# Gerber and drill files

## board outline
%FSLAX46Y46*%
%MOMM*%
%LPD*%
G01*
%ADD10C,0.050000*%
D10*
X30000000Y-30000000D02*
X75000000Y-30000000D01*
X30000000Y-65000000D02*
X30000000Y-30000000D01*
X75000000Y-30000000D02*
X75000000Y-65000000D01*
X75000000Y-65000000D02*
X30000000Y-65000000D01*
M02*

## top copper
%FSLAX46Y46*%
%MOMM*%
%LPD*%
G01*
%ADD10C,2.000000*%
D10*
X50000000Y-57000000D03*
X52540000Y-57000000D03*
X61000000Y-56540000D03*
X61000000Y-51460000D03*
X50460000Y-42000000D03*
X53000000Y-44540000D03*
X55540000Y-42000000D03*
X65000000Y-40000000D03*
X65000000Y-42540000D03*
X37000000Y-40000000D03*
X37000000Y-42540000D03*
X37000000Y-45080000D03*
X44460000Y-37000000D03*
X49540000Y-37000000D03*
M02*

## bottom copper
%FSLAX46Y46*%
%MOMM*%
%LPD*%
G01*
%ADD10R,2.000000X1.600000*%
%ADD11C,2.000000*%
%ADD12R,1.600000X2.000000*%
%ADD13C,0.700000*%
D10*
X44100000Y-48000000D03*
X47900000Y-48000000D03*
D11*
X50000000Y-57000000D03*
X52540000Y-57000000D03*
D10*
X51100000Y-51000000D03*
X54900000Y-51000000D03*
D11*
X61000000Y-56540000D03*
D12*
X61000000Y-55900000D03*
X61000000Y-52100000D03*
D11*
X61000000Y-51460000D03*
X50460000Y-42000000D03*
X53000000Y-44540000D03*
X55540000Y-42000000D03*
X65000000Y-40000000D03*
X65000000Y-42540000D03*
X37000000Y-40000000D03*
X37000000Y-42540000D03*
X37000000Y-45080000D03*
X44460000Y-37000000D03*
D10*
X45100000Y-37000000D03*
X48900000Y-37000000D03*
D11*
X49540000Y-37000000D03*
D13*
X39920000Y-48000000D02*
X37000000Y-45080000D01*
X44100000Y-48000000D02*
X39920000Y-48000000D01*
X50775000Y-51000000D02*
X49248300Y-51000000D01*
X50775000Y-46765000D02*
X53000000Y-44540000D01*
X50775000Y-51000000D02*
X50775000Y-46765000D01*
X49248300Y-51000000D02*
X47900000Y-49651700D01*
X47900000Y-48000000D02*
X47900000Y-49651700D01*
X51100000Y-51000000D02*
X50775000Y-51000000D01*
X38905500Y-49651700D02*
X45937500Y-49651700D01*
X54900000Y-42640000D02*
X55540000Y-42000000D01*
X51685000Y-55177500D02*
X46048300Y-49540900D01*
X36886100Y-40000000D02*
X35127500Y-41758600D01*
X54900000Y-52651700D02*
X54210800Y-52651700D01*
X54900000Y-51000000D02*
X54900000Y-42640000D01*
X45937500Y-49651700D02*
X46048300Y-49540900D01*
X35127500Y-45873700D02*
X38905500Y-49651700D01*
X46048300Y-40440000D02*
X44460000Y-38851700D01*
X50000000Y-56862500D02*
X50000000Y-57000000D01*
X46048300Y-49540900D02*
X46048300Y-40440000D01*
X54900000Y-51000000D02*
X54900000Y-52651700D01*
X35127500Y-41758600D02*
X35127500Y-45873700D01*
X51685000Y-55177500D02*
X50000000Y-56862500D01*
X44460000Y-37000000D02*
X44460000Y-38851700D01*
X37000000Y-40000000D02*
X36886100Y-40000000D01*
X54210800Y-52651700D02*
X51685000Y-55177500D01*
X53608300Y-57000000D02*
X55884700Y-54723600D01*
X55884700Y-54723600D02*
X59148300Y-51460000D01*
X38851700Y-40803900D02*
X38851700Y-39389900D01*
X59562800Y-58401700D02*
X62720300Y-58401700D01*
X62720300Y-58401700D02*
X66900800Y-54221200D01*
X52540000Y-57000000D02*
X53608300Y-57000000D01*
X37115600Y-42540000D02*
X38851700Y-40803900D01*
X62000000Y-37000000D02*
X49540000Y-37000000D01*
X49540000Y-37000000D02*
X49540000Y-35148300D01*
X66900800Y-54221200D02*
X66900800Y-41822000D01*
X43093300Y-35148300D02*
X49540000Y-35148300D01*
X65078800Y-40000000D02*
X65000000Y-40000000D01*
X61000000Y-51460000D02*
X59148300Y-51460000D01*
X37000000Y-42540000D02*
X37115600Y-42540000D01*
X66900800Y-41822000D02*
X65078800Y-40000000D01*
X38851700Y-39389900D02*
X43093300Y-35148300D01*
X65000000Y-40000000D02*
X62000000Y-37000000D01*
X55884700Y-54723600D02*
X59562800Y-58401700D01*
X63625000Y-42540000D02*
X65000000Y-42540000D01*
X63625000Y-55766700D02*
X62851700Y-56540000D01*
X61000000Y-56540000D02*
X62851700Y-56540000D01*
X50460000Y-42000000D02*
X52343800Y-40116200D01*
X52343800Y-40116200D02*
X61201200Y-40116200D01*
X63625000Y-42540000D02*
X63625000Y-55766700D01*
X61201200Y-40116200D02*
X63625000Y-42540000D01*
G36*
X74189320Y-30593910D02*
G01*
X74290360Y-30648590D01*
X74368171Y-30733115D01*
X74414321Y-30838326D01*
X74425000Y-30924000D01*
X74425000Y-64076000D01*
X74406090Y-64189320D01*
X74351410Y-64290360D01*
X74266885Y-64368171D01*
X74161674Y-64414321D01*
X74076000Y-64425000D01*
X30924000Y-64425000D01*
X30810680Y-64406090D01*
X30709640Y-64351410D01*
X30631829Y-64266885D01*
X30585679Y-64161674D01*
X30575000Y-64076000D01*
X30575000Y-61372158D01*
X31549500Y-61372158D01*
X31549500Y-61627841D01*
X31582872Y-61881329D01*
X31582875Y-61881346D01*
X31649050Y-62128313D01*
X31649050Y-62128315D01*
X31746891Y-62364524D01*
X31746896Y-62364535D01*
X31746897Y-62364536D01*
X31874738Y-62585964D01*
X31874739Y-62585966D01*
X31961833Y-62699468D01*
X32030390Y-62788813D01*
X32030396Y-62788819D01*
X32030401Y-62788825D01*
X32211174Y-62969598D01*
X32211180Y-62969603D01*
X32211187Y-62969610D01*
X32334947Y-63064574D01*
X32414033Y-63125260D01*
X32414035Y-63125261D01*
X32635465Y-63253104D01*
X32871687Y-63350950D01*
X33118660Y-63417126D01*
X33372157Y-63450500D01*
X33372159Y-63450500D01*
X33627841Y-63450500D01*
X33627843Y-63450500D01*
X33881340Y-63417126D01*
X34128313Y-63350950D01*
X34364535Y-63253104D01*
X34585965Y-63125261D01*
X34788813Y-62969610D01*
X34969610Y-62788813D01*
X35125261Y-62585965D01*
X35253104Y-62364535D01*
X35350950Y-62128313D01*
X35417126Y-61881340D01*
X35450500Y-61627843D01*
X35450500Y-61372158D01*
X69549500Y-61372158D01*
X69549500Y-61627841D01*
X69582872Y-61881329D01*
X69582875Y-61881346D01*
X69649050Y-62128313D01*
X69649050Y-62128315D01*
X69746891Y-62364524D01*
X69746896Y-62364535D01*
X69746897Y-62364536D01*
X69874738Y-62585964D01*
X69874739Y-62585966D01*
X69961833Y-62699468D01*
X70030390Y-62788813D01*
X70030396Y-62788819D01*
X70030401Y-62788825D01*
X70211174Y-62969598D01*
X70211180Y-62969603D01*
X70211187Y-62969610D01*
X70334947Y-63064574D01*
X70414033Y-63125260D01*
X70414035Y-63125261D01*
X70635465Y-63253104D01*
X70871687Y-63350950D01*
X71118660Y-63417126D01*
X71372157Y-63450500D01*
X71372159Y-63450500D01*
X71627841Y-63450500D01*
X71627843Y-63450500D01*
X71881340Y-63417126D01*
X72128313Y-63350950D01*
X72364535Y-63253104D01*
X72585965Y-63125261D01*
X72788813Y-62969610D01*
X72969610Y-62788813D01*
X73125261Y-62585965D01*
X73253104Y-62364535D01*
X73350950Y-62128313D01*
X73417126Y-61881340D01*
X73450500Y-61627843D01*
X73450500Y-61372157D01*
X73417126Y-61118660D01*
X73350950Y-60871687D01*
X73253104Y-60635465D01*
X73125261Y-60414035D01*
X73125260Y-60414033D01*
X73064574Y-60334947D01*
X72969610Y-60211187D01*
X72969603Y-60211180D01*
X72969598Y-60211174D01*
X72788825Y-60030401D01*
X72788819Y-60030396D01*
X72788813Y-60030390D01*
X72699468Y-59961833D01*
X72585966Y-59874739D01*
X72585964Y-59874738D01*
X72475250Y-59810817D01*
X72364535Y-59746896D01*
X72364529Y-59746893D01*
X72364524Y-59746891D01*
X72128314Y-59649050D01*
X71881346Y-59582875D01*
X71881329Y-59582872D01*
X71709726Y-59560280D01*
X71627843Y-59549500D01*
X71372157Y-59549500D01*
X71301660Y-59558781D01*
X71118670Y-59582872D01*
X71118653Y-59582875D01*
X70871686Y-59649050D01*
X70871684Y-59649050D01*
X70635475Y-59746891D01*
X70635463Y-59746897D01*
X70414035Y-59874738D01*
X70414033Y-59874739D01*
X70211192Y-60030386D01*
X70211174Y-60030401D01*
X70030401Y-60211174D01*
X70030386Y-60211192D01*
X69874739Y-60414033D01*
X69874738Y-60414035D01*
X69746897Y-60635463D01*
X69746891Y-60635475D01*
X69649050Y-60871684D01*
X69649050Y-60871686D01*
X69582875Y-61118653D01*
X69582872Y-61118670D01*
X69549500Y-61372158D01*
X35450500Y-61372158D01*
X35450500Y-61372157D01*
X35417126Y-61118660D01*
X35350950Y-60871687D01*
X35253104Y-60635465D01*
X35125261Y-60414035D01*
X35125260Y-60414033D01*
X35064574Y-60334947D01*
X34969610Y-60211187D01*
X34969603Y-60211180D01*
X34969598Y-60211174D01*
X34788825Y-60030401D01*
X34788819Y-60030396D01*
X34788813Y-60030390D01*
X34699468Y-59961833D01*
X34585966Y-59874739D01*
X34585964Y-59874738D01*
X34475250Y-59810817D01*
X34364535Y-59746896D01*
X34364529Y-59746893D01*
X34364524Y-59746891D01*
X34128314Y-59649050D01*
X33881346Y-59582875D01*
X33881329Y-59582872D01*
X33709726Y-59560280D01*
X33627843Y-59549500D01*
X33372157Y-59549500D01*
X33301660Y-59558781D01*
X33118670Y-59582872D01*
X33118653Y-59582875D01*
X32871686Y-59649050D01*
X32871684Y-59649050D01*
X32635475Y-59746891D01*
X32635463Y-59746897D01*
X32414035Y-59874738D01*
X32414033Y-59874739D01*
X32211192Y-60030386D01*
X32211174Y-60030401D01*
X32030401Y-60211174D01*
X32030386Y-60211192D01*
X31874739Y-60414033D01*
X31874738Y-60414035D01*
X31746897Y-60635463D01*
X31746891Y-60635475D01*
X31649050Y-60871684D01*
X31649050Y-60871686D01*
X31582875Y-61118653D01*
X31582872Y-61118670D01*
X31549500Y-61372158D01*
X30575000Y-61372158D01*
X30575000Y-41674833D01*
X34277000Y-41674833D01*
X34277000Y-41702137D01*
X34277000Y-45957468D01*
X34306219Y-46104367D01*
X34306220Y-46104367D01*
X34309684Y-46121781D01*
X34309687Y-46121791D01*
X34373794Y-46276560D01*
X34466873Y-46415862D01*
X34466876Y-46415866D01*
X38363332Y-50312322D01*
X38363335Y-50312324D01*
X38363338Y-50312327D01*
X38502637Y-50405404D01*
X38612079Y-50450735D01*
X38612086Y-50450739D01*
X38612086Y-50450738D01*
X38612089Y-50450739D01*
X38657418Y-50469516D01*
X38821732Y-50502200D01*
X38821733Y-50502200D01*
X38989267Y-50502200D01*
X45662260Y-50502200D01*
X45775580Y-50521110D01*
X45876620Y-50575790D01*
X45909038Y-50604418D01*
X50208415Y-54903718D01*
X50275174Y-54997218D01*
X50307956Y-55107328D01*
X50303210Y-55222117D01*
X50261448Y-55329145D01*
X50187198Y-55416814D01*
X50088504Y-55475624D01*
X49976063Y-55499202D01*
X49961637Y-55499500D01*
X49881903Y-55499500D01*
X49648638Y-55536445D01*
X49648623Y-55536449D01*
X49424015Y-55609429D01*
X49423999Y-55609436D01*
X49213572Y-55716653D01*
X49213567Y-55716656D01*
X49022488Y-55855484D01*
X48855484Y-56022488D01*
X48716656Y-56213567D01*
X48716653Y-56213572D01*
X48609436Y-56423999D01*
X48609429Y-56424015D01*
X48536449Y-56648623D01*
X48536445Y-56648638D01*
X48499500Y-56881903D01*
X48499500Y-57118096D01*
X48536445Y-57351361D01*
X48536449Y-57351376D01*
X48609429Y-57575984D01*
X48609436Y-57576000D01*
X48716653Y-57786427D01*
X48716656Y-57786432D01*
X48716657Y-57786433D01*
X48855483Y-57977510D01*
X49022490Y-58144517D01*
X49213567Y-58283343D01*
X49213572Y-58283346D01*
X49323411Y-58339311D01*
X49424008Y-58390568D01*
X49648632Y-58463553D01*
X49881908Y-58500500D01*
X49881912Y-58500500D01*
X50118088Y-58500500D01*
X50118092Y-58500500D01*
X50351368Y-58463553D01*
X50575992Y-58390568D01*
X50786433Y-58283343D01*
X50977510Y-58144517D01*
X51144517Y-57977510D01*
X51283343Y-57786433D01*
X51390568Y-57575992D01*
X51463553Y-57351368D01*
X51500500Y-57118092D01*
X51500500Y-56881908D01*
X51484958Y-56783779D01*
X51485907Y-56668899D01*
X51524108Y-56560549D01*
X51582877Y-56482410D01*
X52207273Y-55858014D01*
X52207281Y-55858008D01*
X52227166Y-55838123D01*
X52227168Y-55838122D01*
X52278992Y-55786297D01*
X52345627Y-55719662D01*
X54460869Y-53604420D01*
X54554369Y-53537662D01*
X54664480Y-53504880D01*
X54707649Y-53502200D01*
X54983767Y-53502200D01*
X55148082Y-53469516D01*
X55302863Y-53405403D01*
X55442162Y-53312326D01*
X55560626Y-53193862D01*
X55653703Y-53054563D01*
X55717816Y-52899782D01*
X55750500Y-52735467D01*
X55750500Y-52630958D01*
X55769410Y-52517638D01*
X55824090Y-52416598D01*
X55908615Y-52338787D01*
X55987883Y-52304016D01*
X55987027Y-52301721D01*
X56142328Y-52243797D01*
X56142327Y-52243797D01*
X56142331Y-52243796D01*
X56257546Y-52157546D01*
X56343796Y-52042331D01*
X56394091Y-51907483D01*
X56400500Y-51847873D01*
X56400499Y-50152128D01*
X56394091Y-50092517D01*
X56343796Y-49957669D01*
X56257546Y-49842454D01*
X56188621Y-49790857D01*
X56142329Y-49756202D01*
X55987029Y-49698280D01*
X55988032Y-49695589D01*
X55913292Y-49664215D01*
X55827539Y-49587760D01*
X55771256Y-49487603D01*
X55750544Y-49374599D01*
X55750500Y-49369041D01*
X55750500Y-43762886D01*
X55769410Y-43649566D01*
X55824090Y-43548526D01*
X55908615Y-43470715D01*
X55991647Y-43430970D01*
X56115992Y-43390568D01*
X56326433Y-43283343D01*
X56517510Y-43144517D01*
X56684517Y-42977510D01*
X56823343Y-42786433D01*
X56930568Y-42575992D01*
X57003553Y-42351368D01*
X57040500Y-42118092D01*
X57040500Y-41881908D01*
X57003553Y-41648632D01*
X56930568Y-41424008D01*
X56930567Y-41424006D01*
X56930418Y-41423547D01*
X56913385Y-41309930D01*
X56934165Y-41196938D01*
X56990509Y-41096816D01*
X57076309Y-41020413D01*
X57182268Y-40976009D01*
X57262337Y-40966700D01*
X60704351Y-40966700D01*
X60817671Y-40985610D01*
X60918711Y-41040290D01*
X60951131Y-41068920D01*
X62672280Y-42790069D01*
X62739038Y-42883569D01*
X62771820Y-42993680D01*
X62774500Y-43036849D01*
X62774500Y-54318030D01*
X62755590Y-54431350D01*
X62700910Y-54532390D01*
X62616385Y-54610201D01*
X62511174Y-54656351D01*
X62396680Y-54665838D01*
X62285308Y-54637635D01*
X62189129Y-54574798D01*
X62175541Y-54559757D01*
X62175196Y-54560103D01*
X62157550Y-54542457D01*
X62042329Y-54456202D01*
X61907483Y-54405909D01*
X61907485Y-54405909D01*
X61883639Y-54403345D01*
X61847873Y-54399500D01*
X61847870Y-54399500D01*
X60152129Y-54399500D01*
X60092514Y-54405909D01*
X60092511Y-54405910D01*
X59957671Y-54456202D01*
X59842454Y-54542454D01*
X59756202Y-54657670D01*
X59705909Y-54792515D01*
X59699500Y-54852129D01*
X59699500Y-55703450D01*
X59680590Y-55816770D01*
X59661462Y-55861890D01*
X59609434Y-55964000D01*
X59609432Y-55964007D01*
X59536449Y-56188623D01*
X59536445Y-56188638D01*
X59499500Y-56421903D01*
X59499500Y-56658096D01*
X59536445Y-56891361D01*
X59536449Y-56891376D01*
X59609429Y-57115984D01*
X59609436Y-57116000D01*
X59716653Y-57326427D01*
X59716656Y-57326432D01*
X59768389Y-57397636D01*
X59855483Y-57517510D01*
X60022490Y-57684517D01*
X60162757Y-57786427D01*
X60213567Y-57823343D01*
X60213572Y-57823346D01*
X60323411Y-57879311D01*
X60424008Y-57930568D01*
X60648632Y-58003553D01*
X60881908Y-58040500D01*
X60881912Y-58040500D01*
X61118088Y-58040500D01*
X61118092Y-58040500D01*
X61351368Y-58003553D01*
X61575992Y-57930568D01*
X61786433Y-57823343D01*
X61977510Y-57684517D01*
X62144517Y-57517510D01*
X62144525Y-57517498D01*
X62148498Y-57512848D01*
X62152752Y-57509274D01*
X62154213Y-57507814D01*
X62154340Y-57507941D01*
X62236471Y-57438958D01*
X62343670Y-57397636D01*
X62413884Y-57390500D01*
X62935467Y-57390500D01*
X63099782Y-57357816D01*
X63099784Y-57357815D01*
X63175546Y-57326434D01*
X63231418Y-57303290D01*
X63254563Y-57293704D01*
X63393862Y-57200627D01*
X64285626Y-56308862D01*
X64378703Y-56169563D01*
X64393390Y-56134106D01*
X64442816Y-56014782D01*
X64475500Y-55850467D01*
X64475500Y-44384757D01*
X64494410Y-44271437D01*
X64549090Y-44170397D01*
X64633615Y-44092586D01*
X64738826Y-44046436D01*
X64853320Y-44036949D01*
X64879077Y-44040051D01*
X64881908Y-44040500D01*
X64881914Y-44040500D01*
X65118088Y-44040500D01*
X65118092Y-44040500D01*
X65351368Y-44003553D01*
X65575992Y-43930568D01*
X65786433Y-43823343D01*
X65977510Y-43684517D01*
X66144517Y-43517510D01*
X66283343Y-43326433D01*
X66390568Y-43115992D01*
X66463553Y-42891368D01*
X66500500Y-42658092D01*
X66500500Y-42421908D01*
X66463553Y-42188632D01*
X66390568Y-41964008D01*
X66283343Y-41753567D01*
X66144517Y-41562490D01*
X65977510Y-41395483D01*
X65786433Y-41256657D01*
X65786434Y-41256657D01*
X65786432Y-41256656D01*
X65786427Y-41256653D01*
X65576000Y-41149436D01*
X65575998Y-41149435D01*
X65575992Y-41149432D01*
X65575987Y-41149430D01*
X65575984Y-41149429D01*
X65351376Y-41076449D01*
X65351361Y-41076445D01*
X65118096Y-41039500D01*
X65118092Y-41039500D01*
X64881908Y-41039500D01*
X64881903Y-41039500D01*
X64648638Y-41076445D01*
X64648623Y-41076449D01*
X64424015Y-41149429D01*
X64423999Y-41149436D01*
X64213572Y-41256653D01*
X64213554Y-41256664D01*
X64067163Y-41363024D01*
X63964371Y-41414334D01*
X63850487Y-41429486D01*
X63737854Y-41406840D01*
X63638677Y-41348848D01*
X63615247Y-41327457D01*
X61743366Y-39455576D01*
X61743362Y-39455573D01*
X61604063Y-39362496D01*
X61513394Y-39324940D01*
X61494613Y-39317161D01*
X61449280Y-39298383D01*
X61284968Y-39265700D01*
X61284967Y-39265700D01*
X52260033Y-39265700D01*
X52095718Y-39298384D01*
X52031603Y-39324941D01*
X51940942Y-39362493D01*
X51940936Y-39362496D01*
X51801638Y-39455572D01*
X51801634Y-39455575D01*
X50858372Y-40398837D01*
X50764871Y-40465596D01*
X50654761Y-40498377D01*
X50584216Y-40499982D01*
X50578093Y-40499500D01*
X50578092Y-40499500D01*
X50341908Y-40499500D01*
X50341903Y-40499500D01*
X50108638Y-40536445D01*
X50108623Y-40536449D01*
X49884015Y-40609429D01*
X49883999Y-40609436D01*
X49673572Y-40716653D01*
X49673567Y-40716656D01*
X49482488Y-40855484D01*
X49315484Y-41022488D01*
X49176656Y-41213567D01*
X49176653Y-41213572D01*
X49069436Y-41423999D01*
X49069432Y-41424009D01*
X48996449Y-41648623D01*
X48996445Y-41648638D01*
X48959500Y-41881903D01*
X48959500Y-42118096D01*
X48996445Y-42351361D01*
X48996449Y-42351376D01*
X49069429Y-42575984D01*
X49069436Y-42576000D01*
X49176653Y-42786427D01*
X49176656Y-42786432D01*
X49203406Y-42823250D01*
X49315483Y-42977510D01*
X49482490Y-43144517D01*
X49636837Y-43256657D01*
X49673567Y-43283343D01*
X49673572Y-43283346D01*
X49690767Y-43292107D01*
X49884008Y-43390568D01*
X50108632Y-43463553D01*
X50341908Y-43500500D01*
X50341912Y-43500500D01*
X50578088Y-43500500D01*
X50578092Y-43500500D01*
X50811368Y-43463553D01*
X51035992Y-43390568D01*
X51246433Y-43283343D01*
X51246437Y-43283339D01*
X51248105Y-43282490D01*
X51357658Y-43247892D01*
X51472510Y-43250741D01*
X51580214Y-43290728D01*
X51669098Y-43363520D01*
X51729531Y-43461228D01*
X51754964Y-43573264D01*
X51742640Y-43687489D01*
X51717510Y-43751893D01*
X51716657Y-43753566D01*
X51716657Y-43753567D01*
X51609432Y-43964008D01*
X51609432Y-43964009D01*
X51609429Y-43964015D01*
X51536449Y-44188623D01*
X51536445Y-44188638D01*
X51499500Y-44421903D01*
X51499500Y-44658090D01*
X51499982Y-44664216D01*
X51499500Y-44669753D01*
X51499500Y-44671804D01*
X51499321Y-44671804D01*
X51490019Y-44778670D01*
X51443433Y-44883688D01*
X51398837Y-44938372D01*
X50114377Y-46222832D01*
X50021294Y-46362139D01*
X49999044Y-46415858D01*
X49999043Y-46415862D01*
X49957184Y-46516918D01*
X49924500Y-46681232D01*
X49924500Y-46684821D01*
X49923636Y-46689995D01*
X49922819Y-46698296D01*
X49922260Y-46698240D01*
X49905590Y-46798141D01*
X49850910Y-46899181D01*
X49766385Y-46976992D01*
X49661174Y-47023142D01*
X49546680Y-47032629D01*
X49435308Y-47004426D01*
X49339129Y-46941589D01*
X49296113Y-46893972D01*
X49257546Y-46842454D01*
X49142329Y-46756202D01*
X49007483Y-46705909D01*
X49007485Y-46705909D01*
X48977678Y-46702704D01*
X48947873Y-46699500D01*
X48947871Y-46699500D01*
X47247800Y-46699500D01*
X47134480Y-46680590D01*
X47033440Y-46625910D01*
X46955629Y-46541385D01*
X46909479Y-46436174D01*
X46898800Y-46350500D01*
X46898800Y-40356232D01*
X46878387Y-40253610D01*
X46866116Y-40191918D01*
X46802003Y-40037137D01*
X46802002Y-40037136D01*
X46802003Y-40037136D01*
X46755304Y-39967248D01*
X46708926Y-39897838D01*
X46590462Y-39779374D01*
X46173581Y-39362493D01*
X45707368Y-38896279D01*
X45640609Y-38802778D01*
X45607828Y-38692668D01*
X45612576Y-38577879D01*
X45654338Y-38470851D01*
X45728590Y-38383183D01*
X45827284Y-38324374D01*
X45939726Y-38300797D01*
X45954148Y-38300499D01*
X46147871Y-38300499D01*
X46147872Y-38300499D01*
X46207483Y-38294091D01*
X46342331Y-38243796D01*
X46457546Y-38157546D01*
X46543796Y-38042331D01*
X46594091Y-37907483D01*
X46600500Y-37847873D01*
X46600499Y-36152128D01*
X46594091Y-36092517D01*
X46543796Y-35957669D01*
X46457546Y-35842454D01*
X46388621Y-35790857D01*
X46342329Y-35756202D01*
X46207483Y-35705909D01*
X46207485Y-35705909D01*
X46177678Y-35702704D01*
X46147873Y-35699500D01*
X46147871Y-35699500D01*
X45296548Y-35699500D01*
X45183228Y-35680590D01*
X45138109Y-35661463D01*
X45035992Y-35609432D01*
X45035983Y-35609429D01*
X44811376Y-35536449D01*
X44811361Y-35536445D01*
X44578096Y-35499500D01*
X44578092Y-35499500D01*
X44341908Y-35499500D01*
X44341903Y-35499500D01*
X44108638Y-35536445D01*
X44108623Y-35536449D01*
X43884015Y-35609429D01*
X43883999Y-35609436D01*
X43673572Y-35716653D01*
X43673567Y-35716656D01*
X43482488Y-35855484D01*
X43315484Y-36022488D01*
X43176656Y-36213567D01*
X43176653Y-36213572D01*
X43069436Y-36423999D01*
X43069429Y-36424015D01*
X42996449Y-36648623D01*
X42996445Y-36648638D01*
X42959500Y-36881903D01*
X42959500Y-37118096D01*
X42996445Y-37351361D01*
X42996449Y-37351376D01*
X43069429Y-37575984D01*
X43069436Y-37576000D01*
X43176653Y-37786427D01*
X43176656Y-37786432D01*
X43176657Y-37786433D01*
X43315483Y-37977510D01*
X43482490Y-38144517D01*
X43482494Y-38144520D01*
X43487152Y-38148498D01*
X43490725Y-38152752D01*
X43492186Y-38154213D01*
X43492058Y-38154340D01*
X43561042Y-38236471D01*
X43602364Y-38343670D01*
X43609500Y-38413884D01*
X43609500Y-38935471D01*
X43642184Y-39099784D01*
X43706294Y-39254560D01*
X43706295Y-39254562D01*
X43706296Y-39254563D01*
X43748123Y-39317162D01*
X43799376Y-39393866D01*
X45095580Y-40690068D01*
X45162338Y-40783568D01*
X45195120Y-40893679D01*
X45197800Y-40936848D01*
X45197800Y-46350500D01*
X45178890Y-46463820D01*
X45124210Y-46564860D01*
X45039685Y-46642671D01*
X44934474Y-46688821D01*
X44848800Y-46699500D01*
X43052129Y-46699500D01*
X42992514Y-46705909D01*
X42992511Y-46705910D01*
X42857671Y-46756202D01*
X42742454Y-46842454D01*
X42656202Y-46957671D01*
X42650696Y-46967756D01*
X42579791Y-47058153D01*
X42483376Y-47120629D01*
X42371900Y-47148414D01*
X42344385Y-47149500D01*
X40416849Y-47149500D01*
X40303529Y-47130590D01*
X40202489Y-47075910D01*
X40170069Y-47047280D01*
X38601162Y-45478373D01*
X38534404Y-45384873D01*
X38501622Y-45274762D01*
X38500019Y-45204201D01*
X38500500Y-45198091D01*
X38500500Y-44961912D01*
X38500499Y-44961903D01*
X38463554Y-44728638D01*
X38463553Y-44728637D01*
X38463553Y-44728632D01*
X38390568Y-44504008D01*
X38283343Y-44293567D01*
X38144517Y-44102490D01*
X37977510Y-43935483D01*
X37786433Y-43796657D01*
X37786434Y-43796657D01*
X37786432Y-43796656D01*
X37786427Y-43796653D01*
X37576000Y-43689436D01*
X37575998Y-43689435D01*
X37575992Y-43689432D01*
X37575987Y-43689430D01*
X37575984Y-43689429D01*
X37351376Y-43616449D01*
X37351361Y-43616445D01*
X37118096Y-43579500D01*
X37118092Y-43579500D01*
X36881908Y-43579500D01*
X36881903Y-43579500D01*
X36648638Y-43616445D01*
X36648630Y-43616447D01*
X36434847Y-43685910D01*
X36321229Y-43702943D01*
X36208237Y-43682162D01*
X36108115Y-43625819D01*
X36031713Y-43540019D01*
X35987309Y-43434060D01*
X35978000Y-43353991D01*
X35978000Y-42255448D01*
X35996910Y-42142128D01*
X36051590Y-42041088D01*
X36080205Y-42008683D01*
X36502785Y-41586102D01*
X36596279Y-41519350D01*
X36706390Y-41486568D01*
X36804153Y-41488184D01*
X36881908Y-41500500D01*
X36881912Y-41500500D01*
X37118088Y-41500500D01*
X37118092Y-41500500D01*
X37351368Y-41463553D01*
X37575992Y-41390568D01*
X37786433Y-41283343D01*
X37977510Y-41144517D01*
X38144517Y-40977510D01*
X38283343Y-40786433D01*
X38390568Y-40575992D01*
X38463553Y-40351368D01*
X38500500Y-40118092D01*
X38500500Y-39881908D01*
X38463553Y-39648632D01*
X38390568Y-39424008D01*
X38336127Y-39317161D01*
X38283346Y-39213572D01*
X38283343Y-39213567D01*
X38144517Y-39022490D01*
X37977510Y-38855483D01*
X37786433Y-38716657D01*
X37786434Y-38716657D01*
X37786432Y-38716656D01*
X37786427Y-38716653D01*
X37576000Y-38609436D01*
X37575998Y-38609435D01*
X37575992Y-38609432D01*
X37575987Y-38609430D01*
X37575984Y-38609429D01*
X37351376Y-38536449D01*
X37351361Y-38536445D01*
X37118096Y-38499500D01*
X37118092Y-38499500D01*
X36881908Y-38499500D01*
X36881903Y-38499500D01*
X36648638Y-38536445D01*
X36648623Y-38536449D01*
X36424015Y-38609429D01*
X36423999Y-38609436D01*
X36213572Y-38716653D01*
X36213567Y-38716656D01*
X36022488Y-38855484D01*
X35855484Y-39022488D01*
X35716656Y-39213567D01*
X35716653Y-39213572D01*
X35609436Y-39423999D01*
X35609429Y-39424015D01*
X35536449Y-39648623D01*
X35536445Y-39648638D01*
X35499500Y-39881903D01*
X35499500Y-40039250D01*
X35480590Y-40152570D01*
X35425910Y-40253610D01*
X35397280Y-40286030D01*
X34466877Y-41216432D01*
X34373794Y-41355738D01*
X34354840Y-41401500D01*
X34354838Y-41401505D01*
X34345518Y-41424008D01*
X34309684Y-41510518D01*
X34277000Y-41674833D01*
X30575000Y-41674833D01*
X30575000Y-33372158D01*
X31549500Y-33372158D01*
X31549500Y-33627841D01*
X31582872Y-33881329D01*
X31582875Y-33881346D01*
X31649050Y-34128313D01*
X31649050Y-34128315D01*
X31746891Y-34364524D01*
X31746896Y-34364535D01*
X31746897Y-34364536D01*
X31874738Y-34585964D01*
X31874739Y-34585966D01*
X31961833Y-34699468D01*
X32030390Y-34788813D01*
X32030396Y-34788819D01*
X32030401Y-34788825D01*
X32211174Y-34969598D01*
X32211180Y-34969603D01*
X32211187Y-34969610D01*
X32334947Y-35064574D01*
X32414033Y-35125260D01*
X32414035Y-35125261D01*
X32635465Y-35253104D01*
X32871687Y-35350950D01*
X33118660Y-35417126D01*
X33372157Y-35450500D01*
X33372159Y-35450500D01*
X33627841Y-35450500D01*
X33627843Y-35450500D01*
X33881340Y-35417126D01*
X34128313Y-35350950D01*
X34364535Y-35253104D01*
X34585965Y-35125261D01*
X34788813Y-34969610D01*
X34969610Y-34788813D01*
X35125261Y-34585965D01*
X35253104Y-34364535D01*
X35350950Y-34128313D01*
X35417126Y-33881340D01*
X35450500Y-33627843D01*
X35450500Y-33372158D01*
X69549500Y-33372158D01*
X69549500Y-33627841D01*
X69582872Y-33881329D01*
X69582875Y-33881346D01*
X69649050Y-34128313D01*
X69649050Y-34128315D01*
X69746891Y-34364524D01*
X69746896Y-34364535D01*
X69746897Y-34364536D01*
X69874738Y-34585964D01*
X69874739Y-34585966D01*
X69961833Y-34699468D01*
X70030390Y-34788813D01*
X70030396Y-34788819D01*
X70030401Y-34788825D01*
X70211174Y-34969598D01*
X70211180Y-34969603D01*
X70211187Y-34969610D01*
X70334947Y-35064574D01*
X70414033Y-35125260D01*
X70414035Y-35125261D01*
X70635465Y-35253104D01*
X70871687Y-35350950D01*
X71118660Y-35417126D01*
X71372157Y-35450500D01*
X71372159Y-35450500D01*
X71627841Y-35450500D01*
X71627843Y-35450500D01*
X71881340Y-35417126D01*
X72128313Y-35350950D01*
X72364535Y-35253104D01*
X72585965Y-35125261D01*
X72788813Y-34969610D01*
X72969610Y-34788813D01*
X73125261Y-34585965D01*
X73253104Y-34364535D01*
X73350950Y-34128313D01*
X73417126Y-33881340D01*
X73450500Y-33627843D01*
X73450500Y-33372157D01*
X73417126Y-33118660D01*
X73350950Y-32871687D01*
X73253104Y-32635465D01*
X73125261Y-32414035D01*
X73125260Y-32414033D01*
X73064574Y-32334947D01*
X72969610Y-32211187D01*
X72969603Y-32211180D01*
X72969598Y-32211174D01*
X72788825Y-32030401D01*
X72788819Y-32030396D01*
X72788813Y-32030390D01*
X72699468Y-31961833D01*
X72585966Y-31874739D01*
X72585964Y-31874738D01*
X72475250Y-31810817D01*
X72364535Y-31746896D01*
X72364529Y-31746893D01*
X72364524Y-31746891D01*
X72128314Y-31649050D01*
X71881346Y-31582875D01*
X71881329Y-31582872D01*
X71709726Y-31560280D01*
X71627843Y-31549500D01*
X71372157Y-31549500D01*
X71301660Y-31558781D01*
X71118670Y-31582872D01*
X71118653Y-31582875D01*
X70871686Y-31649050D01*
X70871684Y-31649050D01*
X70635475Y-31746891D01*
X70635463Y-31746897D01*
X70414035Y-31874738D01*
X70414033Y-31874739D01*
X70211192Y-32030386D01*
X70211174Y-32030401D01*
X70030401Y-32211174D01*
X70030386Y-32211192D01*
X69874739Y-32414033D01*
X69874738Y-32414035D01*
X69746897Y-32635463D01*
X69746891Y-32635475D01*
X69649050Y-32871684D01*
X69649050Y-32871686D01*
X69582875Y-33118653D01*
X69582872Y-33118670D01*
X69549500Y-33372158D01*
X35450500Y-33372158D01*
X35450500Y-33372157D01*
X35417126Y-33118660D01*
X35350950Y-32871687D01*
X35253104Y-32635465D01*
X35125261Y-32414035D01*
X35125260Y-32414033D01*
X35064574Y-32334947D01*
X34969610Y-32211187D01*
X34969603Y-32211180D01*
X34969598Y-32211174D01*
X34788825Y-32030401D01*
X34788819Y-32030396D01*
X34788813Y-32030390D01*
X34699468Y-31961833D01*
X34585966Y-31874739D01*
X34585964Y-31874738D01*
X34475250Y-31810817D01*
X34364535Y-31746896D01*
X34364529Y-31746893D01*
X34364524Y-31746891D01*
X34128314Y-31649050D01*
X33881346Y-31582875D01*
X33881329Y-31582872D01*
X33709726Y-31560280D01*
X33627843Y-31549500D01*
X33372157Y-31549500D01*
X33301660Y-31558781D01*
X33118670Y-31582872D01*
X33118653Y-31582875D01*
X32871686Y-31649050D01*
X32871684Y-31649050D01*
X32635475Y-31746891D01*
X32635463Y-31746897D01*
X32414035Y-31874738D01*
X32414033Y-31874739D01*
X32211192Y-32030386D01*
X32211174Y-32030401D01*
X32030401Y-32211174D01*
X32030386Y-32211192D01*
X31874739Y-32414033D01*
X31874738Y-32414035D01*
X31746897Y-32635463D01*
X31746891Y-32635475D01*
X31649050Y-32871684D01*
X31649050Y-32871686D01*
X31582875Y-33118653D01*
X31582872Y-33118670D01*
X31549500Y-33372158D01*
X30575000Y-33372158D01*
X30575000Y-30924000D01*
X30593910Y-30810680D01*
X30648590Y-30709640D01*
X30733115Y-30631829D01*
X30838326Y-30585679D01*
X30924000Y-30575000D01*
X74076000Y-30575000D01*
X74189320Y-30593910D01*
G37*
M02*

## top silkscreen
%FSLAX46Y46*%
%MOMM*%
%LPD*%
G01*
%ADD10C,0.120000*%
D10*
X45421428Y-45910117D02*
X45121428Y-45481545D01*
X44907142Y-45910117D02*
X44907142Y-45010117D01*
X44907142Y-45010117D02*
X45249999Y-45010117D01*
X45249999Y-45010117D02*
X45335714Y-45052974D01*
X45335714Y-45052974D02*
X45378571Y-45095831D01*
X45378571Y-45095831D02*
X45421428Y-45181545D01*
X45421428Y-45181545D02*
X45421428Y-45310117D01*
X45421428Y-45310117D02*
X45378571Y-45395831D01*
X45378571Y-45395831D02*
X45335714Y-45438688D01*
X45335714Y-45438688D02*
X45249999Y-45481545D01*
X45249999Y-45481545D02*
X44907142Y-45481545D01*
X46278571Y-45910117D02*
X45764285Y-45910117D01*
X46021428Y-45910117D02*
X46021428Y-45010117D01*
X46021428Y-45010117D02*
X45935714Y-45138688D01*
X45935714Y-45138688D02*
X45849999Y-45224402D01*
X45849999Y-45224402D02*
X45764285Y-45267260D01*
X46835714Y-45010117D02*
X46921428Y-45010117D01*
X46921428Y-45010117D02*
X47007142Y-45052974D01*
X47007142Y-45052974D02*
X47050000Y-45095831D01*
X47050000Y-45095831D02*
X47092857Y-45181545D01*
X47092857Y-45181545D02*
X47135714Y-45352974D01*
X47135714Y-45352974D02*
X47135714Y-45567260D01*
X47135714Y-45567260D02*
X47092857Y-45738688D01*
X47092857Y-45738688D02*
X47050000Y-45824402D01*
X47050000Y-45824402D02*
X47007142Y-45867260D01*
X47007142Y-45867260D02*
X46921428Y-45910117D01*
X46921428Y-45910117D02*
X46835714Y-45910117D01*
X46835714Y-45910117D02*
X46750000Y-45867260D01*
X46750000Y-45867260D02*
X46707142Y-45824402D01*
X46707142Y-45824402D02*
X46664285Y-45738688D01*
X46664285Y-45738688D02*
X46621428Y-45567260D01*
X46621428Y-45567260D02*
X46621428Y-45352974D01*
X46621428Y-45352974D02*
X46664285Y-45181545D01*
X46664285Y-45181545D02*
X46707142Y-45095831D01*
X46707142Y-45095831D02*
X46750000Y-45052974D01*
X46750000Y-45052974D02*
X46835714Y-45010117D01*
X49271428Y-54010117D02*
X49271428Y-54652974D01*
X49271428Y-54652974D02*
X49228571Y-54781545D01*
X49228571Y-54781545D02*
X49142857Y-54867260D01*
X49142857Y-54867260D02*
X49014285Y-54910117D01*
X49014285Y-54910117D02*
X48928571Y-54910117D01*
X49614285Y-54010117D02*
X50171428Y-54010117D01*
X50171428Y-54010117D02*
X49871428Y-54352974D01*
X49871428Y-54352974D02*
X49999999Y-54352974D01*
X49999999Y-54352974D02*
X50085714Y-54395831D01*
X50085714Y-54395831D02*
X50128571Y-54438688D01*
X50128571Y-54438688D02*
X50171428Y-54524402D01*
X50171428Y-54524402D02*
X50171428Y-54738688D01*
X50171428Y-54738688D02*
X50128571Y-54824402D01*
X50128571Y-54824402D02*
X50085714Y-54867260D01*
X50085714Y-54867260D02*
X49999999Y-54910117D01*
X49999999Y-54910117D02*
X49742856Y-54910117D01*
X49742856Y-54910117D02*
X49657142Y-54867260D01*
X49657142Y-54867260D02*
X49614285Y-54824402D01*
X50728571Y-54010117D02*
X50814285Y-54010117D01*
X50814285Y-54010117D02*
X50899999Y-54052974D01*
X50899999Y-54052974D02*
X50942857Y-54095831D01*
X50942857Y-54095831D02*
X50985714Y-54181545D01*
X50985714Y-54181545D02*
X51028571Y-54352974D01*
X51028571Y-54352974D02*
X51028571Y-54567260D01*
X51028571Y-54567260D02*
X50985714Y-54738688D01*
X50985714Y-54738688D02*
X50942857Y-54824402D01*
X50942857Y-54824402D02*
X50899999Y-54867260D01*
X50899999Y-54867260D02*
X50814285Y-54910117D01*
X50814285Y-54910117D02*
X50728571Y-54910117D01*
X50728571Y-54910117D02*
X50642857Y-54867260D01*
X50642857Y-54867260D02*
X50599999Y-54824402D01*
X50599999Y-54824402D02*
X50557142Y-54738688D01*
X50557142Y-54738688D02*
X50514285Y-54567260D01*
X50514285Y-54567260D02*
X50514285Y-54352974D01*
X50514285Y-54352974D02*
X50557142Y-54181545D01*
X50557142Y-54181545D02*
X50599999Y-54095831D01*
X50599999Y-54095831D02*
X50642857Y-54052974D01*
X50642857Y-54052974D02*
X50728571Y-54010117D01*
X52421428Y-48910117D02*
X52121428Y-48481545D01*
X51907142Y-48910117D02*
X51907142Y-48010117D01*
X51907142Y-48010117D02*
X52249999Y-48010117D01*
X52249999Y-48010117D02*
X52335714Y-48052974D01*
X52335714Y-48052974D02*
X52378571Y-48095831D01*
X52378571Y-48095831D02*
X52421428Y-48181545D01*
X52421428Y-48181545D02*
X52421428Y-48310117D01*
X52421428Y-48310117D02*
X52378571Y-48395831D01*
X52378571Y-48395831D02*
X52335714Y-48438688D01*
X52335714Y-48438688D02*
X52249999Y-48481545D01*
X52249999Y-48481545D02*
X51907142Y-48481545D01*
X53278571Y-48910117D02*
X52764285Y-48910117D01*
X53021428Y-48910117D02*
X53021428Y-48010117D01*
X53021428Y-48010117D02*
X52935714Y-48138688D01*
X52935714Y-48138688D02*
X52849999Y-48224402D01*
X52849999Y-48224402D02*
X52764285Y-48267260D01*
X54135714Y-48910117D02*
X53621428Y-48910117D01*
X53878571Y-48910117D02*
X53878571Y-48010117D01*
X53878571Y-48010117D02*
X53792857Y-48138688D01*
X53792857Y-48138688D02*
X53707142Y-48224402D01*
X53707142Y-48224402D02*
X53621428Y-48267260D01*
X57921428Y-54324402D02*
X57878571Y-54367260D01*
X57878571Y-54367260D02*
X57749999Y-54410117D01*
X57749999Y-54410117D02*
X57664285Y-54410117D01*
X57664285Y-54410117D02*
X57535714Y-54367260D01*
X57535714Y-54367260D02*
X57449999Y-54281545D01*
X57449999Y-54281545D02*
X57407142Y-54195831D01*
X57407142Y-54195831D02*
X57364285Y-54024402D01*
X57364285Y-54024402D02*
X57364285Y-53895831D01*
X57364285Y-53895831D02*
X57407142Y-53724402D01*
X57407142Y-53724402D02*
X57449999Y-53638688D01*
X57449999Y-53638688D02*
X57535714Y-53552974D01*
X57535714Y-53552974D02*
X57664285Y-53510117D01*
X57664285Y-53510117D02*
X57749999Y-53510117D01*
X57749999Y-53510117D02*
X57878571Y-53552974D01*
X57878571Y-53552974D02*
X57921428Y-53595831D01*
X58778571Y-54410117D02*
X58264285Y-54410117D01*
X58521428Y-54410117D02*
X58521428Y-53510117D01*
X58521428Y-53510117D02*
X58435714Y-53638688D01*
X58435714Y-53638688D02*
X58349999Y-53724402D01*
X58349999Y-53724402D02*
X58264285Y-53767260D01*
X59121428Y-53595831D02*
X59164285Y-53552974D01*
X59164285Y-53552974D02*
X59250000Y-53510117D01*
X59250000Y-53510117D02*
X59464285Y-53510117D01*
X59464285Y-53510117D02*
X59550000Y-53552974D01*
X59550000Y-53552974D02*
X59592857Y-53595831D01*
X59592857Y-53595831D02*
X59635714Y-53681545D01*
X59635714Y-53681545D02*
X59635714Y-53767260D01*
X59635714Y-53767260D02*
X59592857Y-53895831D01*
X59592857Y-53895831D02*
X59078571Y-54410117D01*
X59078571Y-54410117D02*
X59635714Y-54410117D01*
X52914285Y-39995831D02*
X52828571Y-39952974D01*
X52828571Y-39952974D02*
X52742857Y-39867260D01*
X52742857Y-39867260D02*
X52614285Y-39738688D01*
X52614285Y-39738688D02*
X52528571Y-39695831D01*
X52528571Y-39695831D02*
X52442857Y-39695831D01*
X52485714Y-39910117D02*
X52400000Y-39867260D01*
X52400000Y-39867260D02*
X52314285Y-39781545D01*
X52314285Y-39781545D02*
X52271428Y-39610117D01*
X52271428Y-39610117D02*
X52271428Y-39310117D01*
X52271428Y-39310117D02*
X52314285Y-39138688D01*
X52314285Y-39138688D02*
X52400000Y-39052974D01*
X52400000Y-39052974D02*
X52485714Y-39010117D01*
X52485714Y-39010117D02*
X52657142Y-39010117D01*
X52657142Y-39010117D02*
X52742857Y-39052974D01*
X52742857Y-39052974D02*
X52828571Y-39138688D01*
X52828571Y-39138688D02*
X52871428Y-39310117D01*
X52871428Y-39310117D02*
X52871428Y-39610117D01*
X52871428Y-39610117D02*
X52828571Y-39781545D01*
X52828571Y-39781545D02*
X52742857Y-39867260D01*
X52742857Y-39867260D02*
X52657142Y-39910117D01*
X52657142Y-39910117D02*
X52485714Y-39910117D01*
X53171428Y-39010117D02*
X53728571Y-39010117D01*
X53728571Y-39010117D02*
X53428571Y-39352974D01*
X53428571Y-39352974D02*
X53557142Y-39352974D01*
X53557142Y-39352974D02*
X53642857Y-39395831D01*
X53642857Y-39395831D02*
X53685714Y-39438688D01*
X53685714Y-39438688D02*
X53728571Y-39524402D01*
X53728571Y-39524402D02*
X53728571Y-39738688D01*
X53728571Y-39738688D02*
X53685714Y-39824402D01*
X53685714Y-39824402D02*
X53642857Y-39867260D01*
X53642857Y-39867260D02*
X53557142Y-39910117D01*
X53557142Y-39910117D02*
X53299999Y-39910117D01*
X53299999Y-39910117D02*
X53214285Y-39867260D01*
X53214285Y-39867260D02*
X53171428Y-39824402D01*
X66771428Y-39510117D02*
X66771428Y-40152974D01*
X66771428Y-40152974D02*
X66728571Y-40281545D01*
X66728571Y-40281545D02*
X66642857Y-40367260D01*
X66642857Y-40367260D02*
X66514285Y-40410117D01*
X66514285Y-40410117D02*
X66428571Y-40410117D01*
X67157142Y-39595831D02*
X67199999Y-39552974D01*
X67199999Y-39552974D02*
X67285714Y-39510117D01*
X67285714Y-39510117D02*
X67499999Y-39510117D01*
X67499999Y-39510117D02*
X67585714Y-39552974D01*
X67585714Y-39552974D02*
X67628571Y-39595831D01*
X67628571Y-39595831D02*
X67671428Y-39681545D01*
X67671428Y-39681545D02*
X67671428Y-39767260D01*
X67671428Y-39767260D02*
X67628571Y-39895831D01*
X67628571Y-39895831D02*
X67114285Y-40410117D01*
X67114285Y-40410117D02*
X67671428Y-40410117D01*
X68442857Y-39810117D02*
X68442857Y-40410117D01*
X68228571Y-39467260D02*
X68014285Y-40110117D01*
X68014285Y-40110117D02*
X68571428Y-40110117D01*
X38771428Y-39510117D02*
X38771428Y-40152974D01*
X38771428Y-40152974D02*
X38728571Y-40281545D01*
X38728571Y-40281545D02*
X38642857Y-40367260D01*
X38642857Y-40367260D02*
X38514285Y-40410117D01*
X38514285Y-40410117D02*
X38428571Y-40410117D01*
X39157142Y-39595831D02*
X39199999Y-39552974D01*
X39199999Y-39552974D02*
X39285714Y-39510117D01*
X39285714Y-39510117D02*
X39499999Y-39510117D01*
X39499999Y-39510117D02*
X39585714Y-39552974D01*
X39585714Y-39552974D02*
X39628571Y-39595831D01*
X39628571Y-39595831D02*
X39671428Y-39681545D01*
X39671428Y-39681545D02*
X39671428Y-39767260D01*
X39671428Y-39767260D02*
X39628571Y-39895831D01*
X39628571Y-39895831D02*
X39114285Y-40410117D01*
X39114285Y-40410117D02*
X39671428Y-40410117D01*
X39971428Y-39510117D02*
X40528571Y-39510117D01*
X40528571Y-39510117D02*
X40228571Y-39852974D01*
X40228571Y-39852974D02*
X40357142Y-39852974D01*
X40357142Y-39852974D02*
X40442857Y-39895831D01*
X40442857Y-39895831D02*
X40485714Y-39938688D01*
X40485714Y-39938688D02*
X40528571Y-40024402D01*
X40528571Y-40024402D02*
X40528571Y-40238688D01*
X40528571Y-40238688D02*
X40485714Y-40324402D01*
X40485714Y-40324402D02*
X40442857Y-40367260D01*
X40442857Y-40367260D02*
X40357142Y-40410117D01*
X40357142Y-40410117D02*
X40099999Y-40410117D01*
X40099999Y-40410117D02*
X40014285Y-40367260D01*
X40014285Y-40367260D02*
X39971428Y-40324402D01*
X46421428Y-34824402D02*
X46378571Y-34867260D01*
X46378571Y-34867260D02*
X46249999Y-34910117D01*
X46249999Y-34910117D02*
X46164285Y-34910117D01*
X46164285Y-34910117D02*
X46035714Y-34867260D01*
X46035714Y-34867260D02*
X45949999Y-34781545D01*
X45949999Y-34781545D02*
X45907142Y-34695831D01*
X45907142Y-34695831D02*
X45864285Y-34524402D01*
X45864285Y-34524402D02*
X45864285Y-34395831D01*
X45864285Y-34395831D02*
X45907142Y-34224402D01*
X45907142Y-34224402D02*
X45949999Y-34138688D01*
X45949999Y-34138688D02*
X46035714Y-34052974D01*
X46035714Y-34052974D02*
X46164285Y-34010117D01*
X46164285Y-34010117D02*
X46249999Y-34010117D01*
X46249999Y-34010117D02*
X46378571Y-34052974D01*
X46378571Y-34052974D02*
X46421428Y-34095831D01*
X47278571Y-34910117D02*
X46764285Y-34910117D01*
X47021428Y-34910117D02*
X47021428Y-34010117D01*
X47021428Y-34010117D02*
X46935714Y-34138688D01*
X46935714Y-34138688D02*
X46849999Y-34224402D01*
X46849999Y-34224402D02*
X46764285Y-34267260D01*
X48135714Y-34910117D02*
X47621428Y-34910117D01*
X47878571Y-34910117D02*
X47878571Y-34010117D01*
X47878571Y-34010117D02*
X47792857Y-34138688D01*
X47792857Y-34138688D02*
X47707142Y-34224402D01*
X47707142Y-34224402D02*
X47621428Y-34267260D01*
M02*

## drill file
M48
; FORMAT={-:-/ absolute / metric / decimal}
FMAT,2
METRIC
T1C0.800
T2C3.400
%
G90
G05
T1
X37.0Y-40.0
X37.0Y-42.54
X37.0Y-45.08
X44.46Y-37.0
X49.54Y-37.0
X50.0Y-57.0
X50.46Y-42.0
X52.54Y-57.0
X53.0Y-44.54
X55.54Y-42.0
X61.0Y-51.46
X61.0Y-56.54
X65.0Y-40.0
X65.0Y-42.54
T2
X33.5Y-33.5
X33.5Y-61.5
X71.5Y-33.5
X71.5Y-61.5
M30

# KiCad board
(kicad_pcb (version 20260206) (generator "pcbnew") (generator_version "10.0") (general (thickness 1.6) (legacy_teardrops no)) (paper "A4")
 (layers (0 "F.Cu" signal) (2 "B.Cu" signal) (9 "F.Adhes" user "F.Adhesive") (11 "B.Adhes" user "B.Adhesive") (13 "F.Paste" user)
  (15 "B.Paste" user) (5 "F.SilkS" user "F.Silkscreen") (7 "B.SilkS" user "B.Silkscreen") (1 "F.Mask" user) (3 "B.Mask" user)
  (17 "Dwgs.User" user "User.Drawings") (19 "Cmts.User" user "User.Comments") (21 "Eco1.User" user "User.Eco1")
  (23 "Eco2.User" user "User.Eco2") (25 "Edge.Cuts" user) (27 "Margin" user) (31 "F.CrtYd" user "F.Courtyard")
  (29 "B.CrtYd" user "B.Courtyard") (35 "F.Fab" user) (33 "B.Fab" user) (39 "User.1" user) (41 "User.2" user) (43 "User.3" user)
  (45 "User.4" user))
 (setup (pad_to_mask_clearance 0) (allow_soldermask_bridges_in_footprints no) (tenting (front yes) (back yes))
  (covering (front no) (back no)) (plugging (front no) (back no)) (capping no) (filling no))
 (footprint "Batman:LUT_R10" (layer "F.Cu") (at 46 48)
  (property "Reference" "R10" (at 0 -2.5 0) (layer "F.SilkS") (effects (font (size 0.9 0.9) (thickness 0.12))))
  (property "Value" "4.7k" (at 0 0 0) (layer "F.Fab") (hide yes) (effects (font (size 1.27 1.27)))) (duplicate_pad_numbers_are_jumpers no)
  (pad "1" smd rect (at -1.9 0) (size 2 1.6) (layers "B.Cu") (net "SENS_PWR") (thermal_bridge_angle 45))
  (pad "2" smd rect (at 1.9 0) (size 2 1.6) (layers "B.Cu") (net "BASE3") (thermal_bridge_angle 45)))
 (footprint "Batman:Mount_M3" (layer "F.Cu") (at 33.5 33.5)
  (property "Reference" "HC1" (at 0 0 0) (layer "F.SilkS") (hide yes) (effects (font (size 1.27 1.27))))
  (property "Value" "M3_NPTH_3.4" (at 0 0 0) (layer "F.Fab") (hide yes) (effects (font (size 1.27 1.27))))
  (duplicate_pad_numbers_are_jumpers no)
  (pad "" np_thru_hole circle (at 0 0) (size 3.4 3.4) (drill 3.4) (layers "*.Cu")))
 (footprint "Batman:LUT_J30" (layer "F.Cu") (at 50 57)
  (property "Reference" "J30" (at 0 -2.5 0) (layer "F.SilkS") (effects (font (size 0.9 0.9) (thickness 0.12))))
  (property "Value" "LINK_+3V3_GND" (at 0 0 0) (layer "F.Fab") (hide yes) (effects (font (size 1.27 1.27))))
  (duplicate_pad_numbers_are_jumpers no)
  (pad "1" thru_hole circle (at 0 0) (size 2 2) (drill 0.8) (layers "*.Cu") (remove_unused_layers no) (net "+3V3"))
  (pad "2" thru_hole circle (at 2.54 0) (size 2 2) (drill 0.8) (layers "*.Cu") (remove_unused_layers no) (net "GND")))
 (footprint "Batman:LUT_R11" (layer "F.Cu") (at 53 51)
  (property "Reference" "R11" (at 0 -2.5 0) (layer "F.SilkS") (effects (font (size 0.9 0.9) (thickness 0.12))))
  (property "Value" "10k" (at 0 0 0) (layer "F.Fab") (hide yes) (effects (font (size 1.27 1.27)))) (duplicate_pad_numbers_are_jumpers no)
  (pad "1" smd rect (at -1.9 0) (size 2 1.6) (layers "B.Cu") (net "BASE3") (thermal_bridge_angle 45))
  (pad "2" smd rect (at 1.9 0) (size 2 1.6) (layers "B.Cu") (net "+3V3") (thermal_bridge_angle 45)))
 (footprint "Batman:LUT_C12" (layer "F.Cu") (at 61 54 90)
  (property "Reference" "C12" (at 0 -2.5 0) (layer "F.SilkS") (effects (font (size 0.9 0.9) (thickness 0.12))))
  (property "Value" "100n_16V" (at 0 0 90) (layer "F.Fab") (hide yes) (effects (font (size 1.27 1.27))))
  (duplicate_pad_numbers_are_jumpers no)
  (pad "1" thru_hole circle (at -2.54 0 90) (size 2 2) (drill 0.8) (layers "*.Cu") (remove_unused_layers no) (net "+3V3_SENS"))
  (pad "1" smd rect (at -1.9 0 90) (size 2 1.6) (layers "B.Cu") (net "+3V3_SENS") (thermal_bridge_angle 45))
  (pad "2" smd rect (at 1.9 0 90) (size 2 1.6) (layers "B.Cu") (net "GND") (thermal_bridge_angle 45))
  (pad "2" thru_hole circle (at 2.54 0 90) (size 2 2) (drill 0.8) (layers "*.Cu") (remove_unused_layers no) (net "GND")))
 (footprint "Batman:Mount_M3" (layer "F.Cu") (at 71.5 33.5)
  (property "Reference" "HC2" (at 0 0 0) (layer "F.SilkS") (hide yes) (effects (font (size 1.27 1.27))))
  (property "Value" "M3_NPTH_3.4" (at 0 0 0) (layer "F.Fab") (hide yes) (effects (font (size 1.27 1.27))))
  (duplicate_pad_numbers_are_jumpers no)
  (pad "" np_thru_hole circle (at 0 0) (size 3.4 3.4) (drill 3.4) (layers "*.Cu")))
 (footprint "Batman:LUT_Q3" (layer "F.Cu") (at 53 42)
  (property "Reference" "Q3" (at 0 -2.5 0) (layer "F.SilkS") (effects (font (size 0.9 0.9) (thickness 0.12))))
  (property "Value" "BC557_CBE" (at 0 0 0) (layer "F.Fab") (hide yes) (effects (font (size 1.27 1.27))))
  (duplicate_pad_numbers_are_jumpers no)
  (pad "1" thru_hole circle (at -2.54 0) (size 2 2) (drill 0.8) (layers "*.Cu") (remove_unused_layers no) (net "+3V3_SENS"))
  (pad "2" thru_hole circle (at 0 2.54) (size 2 2) (drill 0.8) (layers "*.Cu") (remove_unused_layers no) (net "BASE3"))
  (pad "3" thru_hole circle (at 2.54 0) (size 2 2) (drill 0.8) (layers "*.Cu") (remove_unused_layers no) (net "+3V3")))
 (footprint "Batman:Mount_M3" (layer "F.Cu") (at 71.5 61.5)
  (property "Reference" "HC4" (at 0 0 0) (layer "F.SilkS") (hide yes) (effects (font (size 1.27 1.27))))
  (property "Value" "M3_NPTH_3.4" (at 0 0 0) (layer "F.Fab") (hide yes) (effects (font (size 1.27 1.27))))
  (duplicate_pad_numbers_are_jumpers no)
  (pad "" np_thru_hole circle (at 0 0) (size 3.4 3.4) (drill 3.4) (layers "*.Cu")))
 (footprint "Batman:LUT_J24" (layer "F.Cu") (at 65 40 -90)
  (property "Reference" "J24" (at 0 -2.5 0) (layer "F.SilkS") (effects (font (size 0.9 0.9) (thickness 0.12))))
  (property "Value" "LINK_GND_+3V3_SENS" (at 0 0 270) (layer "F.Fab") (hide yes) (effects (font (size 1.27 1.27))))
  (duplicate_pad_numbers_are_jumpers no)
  (pad "1" thru_hole circle (at 0 0 270) (size 2 2) (drill 0.8) (layers "*.Cu") (remove_unused_layers no) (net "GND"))
  (pad "2" thru_hole circle (at 2.54 0 270) (size 2 2) (drill 0.8) (layers "*.Cu") (remove_unused_layers no) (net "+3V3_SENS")))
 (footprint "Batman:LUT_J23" (layer "F.Cu") (at 37 40 -90)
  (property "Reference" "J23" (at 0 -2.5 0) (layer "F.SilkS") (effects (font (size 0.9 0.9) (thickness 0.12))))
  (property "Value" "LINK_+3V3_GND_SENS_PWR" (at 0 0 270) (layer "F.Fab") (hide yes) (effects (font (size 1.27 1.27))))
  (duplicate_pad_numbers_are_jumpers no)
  (pad "1" thru_hole circle (at 0 0 270) (size 2 2) (drill 0.8) (layers "*.Cu") (remove_unused_layers no) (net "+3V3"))
  (pad "2" thru_hole circle (at 2.54 0 270) (size 2 2) (drill 0.8) (layers "*.Cu") (remove_unused_layers no) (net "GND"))
  (pad "3" thru_hole circle (at 5.08 0 270) (size 2 2) (drill 0.8) (layers "*.Cu") (remove_unused_layers no) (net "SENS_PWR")))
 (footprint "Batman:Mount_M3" (layer "F.Cu") (at 33.5 61.5)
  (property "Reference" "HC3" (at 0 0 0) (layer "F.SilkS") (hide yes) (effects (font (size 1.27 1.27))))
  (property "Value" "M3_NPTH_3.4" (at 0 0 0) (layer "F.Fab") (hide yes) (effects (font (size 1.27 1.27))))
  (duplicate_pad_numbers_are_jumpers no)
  (pad "" np_thru_hole circle (at 0 0) (size 3.4 3.4) (drill 3.4) (layers "*.Cu")))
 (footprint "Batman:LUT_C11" (layer "F.Cu") (at 47 37)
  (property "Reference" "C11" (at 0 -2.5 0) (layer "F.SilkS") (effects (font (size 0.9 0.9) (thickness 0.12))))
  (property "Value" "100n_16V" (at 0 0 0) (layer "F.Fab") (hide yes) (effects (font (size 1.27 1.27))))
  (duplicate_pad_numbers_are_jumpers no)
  (pad "1" thru_hole circle (at -2.54 0) (size 2 2) (drill 0.8) (layers "*.Cu") (remove_unused_layers no) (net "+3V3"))
  (pad "1" smd rect (at -1.9 0) (size 2 1.6) (layers "B.Cu") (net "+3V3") (thermal_bridge_angle 45))
  (pad "2" smd rect (at 1.9 0) (size 2 1.6) (layers "B.Cu") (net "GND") (thermal_bridge_angle 45))
  (pad "2" thru_hole circle (at 2.54 0) (size 2 2) (drill 0.8) (layers "*.Cu") (remove_unused_layers no) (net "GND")))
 (gr_line (start 30 30) (end 75 30) (stroke (width 0.05) (type default)) (layer "Edge.Cuts"))
 (gr_line (start 30 65) (end 30 30) (stroke (width 0.05) (type default)) (layer "Edge.Cuts"))
 (gr_line (start 75 30) (end 75 65) (stroke (width 0.05) (type default)) (layer "Edge.Cuts"))
 (gr_line (start 75 65) (end 30 65) (stroke (width 0.05) (type default)) (layer "Edge.Cuts"))
 (segment (start 39.92 48) (end 37 45.08) (width 0.7) (layer "B.Cu") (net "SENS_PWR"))
 (segment (start 44.1 48) (end 39.92 48) (width 0.7) (layer "B.Cu") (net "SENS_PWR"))
 (segment (start 50.775 51) (end 49.2483 51) (width 0.7) (layer "B.Cu") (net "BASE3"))
 (segment (start 50.775 46.765) (end 53 44.54) (width 0.7) (layer "B.Cu") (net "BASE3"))
 (segment (start 50.775 51) (end 50.775 46.765) (width 0.7) (layer "B.Cu") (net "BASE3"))
 (segment (start 49.2483 51) (end 47.9 49.6517) (width 0.7) (layer "B.Cu") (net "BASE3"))
 (segment (start 47.9 48) (end 47.9 49.6517) (width 0.7) (layer "B.Cu") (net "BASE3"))
 (segment (start 51.1 51) (end 50.775 51) (width 0.7) (layer "B.Cu") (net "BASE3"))
 (segment (start 38.9055 49.6517) (end 45.9375 49.6517) (width 0.7) (layer "B.Cu") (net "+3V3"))
 (segment (start 54.9 42.64) (end 55.54 42) (width 0.7) (layer "B.Cu") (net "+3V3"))
 (segment (start 51.685 55.1775) (end 46.0483 49.5409) (width 0.7) (layer "B.Cu") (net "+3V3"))
 (segment (start 36.8861 40) (end 35.1275 41.7586) (width 0.7) (layer "B.Cu") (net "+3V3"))
 (segment (start 54.9 52.6517) (end 54.2108 52.6517) (width 0.7) (layer "B.Cu") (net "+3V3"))
 (segment (start 54.9 51) (end 54.9 42.64) (width 0.7) (layer "B.Cu") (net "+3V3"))
 (segment (start 45.9375 49.6517) (end 46.0483 49.5409) (width 0.7) (layer "B.Cu") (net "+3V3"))
 (segment (start 35.1275 45.8737) (end 38.9055 49.6517) (width 0.7) (layer "B.Cu") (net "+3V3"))
 (segment (start 46.0483 40.44) (end 44.46 38.8517) (width 0.7) (layer "B.Cu") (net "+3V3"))
 (segment (start 50 56.8625) (end 50 57) (width 0.7) (layer "B.Cu") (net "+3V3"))
 (segment (start 46.0483 49.5409) (end 46.0483 40.44) (width 0.7) (layer "B.Cu") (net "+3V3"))
 (segment (start 54.9 51) (end 54.9 52.6517) (width 0.7) (layer "B.Cu") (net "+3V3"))
 (segment (start 35.1275 41.7586) (end 35.1275 45.8737) (width 0.7) (layer "B.Cu") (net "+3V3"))
 (segment (start 51.685 55.1775) (end 50 56.8625) (width 0.7) (layer "B.Cu") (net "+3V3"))
 (segment (start 44.46 37) (end 44.46 38.8517) (width 0.7) (layer "B.Cu") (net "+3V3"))
 (segment (start 37 40) (end 36.8861 40) (width 0.7) (layer "B.Cu") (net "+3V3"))
 (segment (start 54.2108 52.6517) (end 51.685 55.1775) (width 0.7) (layer "B.Cu") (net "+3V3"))
 (segment (start 53.6083 57) (end 55.8847 54.7236) (width 0.7) (layer "B.Cu") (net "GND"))
 (segment (start 55.8847 54.7236) (end 59.1483 51.46) (width 0.7) (layer "B.Cu") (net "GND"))
 (segment (start 38.8517 40.8039) (end 38.8517 39.3899) (width 0.7) (layer "B.Cu") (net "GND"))
 (segment (start 59.5628 58.4017) (end 62.7203 58.4017) (width 0.7) (layer "B.Cu") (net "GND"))
 (segment (start 62.7203 58.4017) (end 66.9008 54.2212) (width 0.7) (layer "B.Cu") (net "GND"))
 (segment (start 52.54 57) (end 53.6083 57) (width 0.7) (layer "B.Cu") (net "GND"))
 (segment (start 37.1156 42.54) (end 38.8517 40.8039) (width 0.7) (layer "B.Cu") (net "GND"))
 (segment (start 62 37) (end 49.54 37) (width 0.7) (layer "B.Cu") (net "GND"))
 (segment (start 49.54 37) (end 49.54 35.1483) (width 0.7) (layer "B.Cu") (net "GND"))
 (segment (start 66.9008 54.2212) (end 66.9008 41.822) (width 0.7) (layer "B.Cu") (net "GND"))
 (segment (start 43.0933 35.1483) (end 49.54 35.1483) (width 0.7) (layer "B.Cu") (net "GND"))
 (segment (start 65.0788 40) (end 65 40) (width 0.7) (layer "B.Cu") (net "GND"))
 (segment (start 61 51.46) (end 59.1483 51.46) (width 0.7) (layer "B.Cu") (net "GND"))
 (segment (start 37 42.54) (end 37.1156 42.54) (width 0.7) (layer "B.Cu") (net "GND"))
 (segment (start 66.9008 41.822) (end 65.0788 40) (width 0.7) (layer "B.Cu") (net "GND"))
 (segment (start 38.8517 39.3899) (end 43.0933 35.1483) (width 0.7) (layer "B.Cu") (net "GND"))
 (segment (start 65 40) (end 62 37) (width 0.7) (layer "B.Cu") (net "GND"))
 (segment (start 55.8847 54.7236) (end 59.5628 58.4017) (width 0.7) (layer "B.Cu") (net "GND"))
 (segment (start 63.625 42.54) (end 65 42.54) (width 0.7) (layer "B.Cu") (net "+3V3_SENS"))
 (segment (start 63.625 55.7667) (end 62.8517 56.54) (width 0.7) (layer "B.Cu") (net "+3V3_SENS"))
 (segment (start 61 56.54) (end 62.8517 56.54) (width 0.7) (layer "B.Cu") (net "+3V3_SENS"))
 (segment (start 50.46 42) (end 52.3438 40.1162) (width 0.7) (layer "B.Cu") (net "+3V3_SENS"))
 (segment (start 52.3438 40.1162) (end 61.2012 40.1162) (width 0.7) (layer "B.Cu") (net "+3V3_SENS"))
 (segment (start 63.625 42.54) (end 63.625 55.7667) (width 0.7) (layer "B.Cu") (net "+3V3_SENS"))
 (segment (start 61.2012 40.1162) (end 63.625 42.54) (width 0.7) (layer "B.Cu") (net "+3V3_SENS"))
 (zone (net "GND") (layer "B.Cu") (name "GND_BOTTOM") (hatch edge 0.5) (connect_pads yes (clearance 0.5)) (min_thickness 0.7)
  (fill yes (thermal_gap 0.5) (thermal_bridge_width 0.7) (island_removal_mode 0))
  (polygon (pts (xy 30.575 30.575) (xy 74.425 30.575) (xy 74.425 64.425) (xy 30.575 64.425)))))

